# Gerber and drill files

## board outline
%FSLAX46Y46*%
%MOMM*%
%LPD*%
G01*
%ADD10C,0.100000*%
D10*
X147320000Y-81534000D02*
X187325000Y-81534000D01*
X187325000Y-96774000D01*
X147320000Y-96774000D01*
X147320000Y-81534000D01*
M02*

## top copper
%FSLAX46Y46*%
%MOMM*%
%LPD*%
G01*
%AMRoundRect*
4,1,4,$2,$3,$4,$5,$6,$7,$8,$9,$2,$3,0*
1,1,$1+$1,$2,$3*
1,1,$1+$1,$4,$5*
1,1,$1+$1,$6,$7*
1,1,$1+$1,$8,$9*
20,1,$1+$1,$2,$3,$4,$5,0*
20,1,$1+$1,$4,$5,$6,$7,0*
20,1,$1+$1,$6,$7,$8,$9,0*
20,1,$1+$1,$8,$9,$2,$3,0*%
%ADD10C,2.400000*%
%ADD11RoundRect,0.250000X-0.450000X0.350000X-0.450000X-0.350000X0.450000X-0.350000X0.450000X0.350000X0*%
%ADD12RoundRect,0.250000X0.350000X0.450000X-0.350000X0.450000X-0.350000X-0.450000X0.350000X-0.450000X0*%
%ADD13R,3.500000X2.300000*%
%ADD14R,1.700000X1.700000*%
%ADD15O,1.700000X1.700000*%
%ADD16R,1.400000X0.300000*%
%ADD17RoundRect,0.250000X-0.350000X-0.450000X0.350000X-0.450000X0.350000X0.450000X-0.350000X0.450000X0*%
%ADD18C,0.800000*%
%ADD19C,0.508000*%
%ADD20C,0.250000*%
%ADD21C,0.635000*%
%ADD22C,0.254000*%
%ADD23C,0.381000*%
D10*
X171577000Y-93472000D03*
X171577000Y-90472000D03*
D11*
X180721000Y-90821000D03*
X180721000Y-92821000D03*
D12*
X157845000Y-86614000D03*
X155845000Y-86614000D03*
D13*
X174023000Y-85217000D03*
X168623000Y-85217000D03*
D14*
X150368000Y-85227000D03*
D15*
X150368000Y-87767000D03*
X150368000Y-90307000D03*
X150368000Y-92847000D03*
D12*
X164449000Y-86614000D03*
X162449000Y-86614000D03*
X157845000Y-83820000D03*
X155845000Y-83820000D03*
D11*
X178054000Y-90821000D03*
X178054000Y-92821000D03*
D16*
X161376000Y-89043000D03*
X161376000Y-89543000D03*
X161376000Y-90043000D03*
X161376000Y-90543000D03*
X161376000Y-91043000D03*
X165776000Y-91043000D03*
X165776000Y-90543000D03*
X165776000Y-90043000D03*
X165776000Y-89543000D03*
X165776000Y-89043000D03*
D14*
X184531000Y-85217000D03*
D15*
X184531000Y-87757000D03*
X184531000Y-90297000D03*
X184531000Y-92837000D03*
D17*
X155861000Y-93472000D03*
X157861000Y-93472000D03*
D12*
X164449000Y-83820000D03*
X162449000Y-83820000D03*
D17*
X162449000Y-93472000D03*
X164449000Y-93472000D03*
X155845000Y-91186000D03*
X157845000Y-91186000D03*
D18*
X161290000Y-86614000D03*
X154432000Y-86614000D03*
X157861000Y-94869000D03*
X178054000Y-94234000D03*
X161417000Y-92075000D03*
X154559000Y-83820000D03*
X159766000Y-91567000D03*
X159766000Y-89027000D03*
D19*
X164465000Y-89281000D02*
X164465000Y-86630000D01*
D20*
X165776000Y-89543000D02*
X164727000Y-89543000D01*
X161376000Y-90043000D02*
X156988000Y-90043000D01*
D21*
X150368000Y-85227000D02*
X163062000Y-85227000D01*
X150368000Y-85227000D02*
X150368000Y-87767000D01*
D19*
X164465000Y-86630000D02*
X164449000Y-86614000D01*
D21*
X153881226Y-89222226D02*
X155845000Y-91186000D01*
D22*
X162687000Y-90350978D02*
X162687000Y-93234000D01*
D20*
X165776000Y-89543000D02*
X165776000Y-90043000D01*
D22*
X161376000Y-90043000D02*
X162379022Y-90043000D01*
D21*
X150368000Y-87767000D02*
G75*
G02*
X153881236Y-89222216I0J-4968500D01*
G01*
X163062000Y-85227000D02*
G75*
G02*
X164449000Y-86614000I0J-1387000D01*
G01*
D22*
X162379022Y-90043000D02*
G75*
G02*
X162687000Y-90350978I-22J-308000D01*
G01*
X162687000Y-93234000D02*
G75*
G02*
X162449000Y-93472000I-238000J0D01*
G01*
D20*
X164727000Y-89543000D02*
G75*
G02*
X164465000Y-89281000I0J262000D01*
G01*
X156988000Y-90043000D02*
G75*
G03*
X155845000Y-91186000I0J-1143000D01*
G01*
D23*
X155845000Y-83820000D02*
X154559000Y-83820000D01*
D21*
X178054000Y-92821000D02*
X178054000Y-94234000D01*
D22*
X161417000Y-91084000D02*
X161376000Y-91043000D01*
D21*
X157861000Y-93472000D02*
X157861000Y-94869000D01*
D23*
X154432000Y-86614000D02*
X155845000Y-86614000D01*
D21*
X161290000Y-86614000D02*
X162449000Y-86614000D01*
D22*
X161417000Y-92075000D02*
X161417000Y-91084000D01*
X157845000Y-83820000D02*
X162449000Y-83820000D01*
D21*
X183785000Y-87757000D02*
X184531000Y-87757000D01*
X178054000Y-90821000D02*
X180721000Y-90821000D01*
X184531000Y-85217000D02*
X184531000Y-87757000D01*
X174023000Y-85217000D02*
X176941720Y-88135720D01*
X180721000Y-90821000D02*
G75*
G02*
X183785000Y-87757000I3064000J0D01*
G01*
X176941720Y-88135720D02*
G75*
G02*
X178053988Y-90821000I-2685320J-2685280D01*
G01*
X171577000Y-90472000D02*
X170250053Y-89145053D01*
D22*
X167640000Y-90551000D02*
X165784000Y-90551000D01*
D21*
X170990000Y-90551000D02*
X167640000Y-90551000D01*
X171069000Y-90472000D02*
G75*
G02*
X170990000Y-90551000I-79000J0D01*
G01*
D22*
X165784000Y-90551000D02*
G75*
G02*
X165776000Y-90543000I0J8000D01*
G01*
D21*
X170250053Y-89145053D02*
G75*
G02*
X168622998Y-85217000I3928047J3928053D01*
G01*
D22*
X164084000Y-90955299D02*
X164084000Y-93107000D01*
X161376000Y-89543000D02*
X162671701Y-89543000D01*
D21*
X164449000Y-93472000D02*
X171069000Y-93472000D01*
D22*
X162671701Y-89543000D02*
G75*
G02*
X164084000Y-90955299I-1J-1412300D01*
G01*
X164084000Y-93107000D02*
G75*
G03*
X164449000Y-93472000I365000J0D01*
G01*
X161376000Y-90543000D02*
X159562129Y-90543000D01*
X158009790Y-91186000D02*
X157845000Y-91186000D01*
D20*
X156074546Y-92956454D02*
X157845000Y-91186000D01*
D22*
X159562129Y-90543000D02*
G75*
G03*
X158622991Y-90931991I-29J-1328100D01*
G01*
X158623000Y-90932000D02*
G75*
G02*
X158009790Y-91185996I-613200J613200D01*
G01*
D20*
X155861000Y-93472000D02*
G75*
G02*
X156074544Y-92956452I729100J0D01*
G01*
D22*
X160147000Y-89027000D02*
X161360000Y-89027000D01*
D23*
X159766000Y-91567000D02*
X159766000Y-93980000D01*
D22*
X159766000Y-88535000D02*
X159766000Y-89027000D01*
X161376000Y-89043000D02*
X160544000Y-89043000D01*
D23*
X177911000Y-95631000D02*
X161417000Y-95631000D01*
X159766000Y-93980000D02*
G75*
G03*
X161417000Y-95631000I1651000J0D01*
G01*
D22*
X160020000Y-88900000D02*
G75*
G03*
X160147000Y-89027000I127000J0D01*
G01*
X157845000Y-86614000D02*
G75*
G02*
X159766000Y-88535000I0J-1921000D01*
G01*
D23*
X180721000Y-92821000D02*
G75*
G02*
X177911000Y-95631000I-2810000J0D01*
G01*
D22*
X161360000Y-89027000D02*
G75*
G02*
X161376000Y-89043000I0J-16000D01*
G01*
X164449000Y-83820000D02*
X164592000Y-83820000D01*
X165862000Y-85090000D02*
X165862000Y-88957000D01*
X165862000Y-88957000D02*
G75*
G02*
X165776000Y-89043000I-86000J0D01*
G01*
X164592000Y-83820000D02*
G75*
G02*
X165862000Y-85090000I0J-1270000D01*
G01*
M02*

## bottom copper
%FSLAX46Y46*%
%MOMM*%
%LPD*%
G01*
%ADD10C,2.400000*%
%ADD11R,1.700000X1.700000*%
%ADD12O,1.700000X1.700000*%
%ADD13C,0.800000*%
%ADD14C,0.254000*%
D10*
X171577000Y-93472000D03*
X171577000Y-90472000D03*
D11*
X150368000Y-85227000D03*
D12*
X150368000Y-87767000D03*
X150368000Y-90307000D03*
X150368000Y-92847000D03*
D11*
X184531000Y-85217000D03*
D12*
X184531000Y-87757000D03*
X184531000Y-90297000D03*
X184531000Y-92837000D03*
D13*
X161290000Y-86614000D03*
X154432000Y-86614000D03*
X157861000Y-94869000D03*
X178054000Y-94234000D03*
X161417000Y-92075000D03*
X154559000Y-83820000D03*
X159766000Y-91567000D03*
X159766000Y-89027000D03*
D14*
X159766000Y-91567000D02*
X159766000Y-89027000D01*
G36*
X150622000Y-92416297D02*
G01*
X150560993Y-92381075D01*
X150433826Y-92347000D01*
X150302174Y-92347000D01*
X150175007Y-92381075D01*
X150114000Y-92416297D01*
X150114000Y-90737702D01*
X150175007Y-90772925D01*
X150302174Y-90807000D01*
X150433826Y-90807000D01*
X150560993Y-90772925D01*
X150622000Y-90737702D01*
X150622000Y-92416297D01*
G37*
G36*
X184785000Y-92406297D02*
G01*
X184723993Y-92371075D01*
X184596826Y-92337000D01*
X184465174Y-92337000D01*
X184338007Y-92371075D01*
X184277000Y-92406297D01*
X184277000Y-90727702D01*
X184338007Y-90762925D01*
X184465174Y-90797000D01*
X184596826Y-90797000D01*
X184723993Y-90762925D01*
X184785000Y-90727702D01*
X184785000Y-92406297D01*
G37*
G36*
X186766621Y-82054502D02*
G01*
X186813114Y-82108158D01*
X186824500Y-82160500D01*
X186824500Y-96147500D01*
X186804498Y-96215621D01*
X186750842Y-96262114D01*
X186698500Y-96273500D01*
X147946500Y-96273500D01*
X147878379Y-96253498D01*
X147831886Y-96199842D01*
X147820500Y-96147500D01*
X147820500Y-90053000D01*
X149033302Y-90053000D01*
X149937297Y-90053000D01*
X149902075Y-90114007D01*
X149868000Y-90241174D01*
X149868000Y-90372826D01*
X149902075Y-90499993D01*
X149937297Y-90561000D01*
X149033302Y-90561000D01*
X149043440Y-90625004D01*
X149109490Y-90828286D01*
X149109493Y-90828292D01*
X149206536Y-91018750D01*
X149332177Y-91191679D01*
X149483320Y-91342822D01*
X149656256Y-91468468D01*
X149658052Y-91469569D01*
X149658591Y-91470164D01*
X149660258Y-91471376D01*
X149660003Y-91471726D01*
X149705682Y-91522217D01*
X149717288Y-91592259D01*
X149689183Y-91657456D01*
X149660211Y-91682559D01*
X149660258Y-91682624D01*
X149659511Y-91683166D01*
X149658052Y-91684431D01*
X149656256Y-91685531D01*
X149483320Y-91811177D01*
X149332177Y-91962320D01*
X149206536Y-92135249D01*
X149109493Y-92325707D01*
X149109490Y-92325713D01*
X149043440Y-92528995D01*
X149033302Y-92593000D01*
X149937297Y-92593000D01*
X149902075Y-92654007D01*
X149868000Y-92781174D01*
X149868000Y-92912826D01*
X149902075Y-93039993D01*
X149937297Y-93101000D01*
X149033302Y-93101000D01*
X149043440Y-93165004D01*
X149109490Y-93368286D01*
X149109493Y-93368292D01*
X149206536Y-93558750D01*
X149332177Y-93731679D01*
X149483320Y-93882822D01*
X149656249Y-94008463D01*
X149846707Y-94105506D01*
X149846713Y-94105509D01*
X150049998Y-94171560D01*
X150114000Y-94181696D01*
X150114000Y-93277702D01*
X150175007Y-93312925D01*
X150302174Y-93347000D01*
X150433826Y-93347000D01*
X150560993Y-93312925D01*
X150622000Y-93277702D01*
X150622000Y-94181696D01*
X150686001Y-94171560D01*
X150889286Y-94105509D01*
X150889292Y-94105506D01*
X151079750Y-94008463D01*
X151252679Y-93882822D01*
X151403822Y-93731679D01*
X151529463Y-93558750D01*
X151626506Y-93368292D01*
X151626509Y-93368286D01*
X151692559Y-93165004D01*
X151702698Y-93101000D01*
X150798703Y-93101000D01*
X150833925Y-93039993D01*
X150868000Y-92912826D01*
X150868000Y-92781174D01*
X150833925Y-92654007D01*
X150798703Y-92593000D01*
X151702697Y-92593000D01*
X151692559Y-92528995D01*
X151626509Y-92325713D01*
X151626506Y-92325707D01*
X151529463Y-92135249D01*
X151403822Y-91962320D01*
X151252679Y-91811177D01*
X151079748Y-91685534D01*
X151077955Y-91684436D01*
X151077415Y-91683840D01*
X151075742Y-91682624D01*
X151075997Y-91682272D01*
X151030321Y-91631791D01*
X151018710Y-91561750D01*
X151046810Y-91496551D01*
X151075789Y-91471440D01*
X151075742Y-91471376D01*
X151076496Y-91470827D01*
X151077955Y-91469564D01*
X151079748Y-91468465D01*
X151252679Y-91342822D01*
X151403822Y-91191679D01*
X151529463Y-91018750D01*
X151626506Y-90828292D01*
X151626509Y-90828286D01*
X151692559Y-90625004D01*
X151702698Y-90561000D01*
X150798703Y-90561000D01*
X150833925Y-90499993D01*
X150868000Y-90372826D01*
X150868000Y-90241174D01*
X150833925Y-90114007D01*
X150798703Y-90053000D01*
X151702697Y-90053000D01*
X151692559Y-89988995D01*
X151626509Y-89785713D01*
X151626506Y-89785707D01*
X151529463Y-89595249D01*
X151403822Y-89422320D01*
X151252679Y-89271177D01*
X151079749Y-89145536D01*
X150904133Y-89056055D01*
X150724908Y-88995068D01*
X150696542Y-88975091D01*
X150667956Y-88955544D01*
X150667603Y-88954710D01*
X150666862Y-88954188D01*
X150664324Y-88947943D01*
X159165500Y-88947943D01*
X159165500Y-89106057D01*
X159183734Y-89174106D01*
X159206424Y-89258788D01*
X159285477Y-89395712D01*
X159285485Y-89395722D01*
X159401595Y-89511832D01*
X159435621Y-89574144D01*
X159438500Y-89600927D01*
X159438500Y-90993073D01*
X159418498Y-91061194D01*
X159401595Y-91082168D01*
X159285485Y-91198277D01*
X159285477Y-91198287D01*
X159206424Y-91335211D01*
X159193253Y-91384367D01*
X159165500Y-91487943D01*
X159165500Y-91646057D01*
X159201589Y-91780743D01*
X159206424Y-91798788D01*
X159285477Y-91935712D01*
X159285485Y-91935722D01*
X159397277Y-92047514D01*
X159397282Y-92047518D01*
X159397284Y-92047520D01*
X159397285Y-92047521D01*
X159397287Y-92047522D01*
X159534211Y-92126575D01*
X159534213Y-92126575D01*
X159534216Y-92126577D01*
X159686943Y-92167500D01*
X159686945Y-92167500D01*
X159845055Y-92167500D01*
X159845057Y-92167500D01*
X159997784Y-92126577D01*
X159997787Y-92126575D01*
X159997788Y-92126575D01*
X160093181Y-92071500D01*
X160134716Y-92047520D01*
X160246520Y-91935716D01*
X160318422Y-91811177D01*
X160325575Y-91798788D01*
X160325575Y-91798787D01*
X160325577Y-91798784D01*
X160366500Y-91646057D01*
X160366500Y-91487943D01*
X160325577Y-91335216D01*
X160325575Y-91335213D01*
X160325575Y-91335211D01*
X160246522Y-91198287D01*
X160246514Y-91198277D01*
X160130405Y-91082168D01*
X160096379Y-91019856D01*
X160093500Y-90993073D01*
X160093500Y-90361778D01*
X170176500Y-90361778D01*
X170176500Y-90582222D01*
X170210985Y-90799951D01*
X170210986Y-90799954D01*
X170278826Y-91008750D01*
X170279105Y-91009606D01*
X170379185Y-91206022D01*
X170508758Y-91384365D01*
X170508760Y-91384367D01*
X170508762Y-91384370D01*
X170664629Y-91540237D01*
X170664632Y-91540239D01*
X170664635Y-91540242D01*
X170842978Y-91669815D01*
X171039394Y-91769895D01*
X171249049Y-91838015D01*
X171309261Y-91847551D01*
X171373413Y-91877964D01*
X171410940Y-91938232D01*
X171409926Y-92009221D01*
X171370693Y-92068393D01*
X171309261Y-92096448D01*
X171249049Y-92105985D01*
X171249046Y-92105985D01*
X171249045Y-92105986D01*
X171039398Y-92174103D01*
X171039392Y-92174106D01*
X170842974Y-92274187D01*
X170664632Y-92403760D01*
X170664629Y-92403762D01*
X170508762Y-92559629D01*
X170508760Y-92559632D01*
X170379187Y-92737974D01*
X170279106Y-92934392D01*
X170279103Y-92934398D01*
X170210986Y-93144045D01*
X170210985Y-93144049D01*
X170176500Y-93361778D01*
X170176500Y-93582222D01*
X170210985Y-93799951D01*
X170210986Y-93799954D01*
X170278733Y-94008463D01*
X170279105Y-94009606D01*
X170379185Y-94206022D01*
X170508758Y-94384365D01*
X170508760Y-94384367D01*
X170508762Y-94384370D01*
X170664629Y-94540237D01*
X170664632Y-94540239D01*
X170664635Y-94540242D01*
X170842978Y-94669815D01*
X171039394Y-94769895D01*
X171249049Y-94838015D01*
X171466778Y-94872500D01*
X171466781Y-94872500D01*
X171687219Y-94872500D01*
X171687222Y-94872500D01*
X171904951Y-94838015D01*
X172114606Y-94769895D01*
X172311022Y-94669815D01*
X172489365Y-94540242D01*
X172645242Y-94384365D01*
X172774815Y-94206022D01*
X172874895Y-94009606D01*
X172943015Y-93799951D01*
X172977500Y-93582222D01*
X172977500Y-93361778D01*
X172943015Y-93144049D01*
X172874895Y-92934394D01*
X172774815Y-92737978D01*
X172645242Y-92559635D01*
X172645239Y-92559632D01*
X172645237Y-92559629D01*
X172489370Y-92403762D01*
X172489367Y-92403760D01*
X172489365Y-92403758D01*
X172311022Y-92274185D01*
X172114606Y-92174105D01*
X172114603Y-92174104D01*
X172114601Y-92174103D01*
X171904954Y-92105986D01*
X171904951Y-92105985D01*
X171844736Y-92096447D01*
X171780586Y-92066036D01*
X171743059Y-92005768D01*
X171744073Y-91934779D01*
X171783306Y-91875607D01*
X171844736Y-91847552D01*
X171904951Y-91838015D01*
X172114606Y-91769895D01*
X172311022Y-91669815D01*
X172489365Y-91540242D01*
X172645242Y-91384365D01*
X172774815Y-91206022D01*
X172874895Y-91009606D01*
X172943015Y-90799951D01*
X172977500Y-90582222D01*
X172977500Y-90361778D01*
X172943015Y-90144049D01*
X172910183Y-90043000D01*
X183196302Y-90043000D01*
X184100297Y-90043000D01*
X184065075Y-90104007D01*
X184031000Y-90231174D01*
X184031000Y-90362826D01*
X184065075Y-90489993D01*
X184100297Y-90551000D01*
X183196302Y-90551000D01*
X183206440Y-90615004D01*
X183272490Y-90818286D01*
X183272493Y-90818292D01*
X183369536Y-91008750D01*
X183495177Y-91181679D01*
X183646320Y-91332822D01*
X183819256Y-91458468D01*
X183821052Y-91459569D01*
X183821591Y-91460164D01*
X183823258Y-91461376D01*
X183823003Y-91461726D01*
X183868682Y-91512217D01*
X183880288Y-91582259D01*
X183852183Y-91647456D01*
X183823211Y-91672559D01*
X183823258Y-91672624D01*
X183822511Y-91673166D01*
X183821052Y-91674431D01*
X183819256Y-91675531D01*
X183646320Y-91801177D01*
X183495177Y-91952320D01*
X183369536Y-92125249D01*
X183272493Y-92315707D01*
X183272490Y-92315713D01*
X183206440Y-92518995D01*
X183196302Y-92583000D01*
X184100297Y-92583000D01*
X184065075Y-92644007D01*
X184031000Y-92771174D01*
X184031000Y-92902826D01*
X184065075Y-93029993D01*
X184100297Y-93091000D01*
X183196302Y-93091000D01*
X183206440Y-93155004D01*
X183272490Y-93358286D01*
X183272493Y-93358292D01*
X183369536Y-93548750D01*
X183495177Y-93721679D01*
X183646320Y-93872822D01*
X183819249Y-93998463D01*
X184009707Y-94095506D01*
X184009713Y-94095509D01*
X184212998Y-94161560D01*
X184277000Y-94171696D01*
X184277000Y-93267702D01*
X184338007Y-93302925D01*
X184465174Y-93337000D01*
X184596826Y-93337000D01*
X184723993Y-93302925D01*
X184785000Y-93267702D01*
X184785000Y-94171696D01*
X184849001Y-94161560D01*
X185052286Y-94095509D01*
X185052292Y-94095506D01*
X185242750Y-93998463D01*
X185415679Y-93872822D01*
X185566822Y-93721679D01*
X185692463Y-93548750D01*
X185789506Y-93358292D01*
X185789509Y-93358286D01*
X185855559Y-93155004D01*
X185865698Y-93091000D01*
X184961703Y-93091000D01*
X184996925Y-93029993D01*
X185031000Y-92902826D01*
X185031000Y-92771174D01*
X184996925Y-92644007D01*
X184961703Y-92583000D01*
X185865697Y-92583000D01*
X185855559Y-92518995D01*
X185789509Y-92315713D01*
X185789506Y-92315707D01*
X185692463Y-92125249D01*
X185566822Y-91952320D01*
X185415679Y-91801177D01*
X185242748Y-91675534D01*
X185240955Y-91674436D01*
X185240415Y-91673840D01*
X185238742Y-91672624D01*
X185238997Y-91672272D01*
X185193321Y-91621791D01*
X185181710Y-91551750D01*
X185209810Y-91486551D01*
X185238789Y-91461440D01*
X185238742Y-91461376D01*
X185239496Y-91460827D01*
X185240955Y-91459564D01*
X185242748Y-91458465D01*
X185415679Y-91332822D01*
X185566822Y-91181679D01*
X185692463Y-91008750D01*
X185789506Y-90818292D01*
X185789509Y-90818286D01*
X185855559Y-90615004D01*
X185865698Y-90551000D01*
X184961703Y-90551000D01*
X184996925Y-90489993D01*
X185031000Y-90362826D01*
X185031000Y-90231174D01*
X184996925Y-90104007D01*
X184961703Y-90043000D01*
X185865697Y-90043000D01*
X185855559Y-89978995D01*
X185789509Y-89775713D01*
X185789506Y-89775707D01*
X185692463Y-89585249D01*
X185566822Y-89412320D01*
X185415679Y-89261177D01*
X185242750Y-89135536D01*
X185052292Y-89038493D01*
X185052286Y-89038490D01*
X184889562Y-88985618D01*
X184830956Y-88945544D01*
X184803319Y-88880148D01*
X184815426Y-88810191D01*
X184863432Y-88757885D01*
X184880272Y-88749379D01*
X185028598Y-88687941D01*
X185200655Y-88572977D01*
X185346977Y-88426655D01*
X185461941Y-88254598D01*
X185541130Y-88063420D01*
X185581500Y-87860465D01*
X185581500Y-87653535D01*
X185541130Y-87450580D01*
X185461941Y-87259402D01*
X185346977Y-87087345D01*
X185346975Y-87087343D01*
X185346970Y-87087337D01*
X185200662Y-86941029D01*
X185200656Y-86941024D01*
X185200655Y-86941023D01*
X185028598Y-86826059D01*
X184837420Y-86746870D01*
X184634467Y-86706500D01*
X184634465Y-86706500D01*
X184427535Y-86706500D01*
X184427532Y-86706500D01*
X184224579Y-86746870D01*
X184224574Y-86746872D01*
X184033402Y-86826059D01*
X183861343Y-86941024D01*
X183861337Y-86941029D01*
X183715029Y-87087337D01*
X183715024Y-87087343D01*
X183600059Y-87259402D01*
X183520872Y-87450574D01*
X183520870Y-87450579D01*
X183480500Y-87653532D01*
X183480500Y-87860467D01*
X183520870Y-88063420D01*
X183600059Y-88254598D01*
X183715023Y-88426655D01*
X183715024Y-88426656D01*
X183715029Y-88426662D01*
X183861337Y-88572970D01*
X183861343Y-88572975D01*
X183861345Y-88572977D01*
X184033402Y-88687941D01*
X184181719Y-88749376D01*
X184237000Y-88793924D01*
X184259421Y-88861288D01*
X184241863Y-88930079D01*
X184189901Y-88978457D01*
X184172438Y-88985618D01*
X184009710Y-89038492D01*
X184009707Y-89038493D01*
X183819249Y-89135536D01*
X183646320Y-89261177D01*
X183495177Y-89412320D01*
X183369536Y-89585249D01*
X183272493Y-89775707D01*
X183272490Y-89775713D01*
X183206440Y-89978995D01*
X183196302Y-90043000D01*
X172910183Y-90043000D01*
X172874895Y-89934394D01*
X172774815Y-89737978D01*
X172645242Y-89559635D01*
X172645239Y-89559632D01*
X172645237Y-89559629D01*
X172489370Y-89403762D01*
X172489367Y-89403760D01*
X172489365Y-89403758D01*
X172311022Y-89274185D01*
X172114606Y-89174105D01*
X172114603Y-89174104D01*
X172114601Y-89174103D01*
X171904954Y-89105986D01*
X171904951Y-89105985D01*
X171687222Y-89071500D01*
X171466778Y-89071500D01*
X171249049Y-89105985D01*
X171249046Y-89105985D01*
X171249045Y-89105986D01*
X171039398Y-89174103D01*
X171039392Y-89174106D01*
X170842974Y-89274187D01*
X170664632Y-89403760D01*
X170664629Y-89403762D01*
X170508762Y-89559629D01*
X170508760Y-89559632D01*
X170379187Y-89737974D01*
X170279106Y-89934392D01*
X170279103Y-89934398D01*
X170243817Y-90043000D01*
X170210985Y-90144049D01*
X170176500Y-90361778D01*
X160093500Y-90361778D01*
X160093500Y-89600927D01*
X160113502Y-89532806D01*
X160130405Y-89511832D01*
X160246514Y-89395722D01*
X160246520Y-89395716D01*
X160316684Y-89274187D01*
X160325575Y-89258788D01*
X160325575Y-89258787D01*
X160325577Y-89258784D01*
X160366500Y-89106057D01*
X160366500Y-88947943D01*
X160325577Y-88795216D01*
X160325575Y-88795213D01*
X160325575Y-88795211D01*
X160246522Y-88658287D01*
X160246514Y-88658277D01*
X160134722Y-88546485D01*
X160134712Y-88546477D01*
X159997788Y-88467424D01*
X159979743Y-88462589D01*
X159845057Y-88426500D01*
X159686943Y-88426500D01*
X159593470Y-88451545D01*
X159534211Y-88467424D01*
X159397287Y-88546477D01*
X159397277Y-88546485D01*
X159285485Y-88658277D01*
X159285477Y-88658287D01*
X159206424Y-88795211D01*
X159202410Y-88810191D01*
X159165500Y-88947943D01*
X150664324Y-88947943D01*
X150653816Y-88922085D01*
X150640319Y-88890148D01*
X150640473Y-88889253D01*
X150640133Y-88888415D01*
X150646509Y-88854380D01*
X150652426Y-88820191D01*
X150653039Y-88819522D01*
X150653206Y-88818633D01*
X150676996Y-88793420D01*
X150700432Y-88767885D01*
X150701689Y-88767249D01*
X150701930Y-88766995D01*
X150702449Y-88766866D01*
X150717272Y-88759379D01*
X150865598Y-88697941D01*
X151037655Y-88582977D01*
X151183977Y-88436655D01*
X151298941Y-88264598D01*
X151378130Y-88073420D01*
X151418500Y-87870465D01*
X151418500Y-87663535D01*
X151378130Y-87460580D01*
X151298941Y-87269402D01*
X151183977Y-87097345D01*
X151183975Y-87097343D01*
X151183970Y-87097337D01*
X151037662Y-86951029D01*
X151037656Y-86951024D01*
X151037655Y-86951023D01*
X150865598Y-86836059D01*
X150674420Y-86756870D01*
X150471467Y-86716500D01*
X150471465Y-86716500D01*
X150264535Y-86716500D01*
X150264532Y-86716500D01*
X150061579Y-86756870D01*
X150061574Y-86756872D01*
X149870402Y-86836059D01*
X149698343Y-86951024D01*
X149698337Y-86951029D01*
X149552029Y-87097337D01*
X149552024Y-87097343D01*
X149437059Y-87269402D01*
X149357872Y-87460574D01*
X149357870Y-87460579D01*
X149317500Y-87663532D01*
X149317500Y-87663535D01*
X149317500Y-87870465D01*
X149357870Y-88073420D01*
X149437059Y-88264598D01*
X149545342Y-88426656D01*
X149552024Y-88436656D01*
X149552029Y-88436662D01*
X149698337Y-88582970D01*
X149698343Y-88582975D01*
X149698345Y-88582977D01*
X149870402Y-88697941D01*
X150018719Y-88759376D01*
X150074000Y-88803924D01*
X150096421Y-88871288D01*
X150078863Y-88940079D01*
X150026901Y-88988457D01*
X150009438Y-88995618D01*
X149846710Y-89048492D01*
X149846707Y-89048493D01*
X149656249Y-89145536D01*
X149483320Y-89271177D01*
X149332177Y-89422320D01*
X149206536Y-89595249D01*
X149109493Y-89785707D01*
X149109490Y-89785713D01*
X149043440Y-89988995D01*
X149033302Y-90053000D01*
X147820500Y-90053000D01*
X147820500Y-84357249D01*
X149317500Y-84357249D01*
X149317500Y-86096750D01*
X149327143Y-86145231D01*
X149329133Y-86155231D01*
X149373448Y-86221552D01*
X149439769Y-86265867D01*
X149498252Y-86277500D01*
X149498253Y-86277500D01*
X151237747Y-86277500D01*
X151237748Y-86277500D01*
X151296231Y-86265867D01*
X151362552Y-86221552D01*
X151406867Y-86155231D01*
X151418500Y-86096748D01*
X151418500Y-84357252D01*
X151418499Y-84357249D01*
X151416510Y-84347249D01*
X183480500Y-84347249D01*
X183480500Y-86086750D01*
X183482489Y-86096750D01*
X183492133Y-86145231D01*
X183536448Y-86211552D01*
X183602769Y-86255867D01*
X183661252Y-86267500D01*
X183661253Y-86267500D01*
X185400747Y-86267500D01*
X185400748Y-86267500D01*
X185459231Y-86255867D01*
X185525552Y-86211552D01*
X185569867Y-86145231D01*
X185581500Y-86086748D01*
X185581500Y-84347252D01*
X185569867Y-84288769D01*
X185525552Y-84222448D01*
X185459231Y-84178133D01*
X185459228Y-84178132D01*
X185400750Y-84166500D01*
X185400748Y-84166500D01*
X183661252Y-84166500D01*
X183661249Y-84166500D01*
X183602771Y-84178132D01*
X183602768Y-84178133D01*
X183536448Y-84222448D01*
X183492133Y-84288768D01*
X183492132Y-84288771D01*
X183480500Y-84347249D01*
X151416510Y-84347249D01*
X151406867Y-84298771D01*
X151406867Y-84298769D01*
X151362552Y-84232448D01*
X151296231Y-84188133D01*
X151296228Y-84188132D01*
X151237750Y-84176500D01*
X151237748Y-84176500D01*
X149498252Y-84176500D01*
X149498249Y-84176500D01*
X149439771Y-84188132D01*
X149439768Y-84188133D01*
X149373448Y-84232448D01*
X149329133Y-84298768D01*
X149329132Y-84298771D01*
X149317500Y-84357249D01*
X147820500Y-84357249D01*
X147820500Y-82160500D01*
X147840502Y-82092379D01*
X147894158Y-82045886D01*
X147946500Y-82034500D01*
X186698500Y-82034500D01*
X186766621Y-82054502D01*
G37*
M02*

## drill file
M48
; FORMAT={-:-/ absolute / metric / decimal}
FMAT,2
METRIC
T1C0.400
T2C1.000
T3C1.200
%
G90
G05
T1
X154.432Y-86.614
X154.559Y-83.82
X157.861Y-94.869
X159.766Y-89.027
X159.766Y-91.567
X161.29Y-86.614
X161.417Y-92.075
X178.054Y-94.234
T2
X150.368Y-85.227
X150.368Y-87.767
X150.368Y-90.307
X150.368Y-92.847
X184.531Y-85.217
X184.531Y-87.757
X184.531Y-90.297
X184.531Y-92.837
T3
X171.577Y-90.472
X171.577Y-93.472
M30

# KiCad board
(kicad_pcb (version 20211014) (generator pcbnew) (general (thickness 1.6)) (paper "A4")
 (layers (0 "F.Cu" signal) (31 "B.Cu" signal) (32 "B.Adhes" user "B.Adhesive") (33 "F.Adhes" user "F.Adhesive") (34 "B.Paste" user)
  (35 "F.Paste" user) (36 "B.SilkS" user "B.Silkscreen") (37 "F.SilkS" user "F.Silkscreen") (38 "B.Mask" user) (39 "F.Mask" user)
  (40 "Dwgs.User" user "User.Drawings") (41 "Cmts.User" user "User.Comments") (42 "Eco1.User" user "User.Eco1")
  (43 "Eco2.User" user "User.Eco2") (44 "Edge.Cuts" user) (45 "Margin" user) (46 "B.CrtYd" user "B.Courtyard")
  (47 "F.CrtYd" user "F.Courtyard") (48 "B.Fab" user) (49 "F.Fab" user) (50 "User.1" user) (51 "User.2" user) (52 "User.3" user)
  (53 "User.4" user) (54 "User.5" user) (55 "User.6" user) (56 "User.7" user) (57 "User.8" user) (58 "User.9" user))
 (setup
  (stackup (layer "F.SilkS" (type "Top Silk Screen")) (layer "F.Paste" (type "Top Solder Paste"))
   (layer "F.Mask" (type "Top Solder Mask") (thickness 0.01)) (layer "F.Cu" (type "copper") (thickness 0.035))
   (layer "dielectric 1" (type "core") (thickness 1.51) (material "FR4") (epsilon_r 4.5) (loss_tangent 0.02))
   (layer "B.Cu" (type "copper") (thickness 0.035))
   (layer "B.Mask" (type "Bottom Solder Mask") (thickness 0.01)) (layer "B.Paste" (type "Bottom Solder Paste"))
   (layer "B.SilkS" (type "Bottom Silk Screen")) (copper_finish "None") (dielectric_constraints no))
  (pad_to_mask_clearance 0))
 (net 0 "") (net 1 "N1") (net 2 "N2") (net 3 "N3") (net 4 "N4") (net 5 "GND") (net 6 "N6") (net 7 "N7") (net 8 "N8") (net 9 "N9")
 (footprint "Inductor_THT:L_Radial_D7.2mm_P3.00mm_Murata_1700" (layer "F.Cu") (at 171.577 93.472 90)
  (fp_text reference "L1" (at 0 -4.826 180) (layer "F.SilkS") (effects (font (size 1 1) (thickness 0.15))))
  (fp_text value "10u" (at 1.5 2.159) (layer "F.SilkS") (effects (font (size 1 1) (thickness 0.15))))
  (pad "1" thru_hole circle (at 0 0 90) (size 2.4 2.4) (drill 1.2) (layers *.Cu *.Mask) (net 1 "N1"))
  (pad "2" thru_hole circle (at 3 0 90) (size 2.4 2.4) (drill 1.2) (layers *.Cu *.Mask) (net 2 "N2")))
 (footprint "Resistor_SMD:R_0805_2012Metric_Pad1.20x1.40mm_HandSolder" (layer "F.Cu") (at 180.721 91.821 -90)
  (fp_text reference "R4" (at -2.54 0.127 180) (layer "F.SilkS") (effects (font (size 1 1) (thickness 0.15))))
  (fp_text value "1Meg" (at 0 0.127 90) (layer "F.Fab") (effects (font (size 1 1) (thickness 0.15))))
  (pad "1" smd roundrect (at -1 0 270) (size 1.2 1.4) (layers "F.Cu" "F.Paste" "F.Mask") (roundrect_rratio 0.208333) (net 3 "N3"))
  (pad "2" smd roundrect (at 1 0 270) (size 1.2 1.4) (layers "F.Cu" "F.Paste" "F.Mask") (roundrect_rratio 0.208333) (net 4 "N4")))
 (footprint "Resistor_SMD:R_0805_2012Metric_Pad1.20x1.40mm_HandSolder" (layer "F.Cu") (at 156.845 86.614 180)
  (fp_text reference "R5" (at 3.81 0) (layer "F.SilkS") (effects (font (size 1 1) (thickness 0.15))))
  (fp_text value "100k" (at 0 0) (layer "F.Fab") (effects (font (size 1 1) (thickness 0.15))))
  (pad "1" smd roundrect (at -1 0 180) (size 1.2 1.4) (layers "F.Cu" "F.Paste" "F.Mask") (roundrect_rratio 0.208333) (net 4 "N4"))
  (pad "2" smd roundrect (at 1 0 180) (size 1.2 1.4) (layers "F.Cu" "F.Paste" "F.Mask") (roundrect_rratio 0.208333) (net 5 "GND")))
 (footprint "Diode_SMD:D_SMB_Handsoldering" (layer "F.Cu") (at 171.323 85.217 180)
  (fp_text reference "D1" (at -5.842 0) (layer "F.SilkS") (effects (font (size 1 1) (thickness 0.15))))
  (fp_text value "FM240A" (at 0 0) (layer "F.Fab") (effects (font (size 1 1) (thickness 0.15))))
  (pad "1" smd rect (at -2.7 0 180) (size 3.5 2.3) (layers "F.Cu" "F.Paste" "F.Mask") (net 3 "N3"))
  (pad "2" smd rect (at 2.7 0 180) (size 3.5 2.3) (layers "F.Cu" "F.Paste" "F.Mask") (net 2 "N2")))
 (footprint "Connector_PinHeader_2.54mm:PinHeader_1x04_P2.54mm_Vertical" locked (layer "F.Cu") (at 150.368 85.227)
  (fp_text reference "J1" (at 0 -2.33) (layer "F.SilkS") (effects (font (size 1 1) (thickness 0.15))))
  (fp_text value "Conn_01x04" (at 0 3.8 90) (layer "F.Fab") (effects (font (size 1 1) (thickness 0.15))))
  (pad "1" thru_hole rect locked (at 0 0) (size 1.7 1.7) (drill 1) (layers *.Cu *.Mask) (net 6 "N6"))
  (pad "2" thru_hole oval locked (at 0 2.54) (size 1.7 1.7) (drill 1) (layers *.Cu *.Mask) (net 6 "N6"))
  (pad "3" thru_hole oval locked (at 0 5.08) (size 1.7 1.7) (drill 1) (layers *.Cu *.Mask) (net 5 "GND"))
  (pad "4" thru_hole oval locked (at 0 7.62) (size 1.7 1.7) (drill 1) (layers *.Cu *.Mask) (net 5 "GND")))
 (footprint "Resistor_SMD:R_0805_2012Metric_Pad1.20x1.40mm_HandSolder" (layer "F.Cu") (at 163.449 86.614 180)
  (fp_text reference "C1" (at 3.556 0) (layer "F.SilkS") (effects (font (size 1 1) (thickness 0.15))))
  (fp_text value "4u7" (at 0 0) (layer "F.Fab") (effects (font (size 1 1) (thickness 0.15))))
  (pad "1" smd roundrect (at -1 0 180) (size 1.2 1.4) (layers "F.Cu" "F.Paste" "F.Mask") (roundrect_rratio 0.208333) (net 6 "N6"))
  (pad "2" smd roundrect (at 1 0 180) (size 1.2 1.4) (layers "F.Cu" "F.Paste" "F.Mask") (roundrect_rratio 0.208333) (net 5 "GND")))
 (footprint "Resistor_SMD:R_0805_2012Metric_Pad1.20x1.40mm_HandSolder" (layer "F.Cu") (at 156.845 83.82 180)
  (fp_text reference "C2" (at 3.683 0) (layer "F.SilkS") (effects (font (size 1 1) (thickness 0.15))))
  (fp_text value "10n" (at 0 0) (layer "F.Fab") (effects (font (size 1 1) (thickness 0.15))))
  (pad "1" smd roundrect (at -1 0 180) (size 1.2 1.4) (layers "F.Cu" "F.Paste" "F.Mask") (roundrect_rratio 0.208333) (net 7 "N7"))
  (pad "2" smd roundrect (at 1 0 180) (size 1.2 1.4) (layers "F.Cu" "F.Paste" "F.Mask") (roundrect_rratio 0.208333) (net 5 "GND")))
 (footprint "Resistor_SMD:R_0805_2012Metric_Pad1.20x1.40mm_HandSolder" (layer "F.Cu") (at 178.054 91.821 -90)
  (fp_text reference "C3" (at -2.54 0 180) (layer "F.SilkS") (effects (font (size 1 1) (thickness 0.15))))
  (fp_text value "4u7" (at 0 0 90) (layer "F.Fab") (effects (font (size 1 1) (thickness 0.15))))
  (pad "1" smd roundrect (at -1 0 270) (size 1.2 1.4) (layers "F.Cu" "F.Paste" "F.Mask") (roundrect_rratio 0.208333) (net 3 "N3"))
  (pad "2" smd roundrect (at 1 0 270) (size 1.2 1.4) (layers "F.Cu" "F.Paste" "F.Mask") (roundrect_rratio 0.208333) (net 5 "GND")))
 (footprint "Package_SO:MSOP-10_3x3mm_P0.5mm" (layer "F.Cu") (at 163.576 90.043)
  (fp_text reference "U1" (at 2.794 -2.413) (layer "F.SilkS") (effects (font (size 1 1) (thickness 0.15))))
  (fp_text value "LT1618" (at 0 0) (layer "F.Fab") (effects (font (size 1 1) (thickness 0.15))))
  (pad "1" smd rect (at -2.2 -1) (size 1.4 0.3) (layers "F.Cu" "F.Paste" "F.Mask") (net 4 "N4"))
  (pad "2" smd rect (at -2.2 -0.5) (size 1.4 0.3) (layers "F.Cu" "F.Paste" "F.Mask") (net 1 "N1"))
  (pad "3" smd rect (at -2.2 0) (size 1.4 0.3) (layers "F.Cu" "F.Paste" "F.Mask") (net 6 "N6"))
  (pad "4" smd rect (at -2.2 0.5) (size 1.4 0.3) (layers "F.Cu" "F.Paste" "F.Mask") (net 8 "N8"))
  (pad "5" smd rect (at -2.2 1) (size 1.4 0.3) (layers "F.Cu" "F.Paste" "F.Mask") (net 5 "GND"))
  (pad "6" smd rect (at 2.2 1) (size 1.4 0.3) (layers "F.Cu" "F.Paste" "F.Mask"))
  (pad "7" smd rect (at 2.2 0.5) (size 1.4 0.3) (layers "F.Cu" "F.Paste" "F.Mask") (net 2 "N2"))
  (pad "8" smd rect (at 2.2 0) (size 1.4 0.3) (layers "F.Cu" "F.Paste" "F.Mask") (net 6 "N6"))
  (pad "9" smd rect (at 2.2 -0.5) (size 1.4 0.3) (layers "F.Cu" "F.Paste" "F.Mask") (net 6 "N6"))
  (pad "10" smd rect (at 2.2 -1) (size 1.4 0.3) (layers "F.Cu" "F.Paste" "F.Mask") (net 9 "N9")))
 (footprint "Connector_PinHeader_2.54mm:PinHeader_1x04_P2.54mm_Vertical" (layer "F.Cu") (at 184.531 85.217)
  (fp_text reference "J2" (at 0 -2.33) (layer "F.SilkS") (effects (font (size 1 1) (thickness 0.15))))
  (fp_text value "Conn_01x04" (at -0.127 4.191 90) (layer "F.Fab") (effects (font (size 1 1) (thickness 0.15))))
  (pad "1" thru_hole rect (at 0 0) (size 1.7 1.7) (drill 1) (layers *.Cu *.Mask) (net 3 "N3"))
  (pad "2" thru_hole oval (at 0 2.54) (size 1.7 1.7) (drill 1) (layers *.Cu *.Mask) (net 3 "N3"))
  (pad "3" thru_hole oval (at 0 5.08) (size 1.7 1.7) (drill 1) (layers *.Cu *.Mask) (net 5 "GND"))
  (pad "4" thru_hole oval (at 0 7.62) (size 1.7 1.7) (drill 1) (layers *.Cu *.Mask) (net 5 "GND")))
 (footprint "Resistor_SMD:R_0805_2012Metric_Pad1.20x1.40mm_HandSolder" (layer "F.Cu") (at 156.861 93.472)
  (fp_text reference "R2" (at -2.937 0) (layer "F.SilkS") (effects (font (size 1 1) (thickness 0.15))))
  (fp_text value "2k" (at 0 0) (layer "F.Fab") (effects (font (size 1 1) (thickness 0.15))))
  (pad "1" smd roundrect (at -1 0) (size 1.2 1.4) (layers "F.Cu" "F.Paste" "F.Mask") (roundrect_rratio 0.208333) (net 8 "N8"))
  (pad "2" smd roundrect (at 1 0) (size 1.2 1.4) (layers "F.Cu" "F.Paste" "F.Mask") (roundrect_rratio 0.208333) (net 5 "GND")))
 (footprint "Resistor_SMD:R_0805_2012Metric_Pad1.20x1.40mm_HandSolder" (layer "F.Cu") (at 163.449 83.82 180)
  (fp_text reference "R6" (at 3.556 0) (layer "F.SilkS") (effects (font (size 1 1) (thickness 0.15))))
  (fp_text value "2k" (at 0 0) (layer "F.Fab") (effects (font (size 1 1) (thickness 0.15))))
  (pad "1" smd roundrect (at -1 0 180) (size 1.2 1.4) (layers "F.Cu" "F.Paste" "F.Mask") (roundrect_rratio 0.208333) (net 9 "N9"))
  (pad "2" smd roundrect (at 1 0 180) (size 1.2 1.4) (layers "F.Cu" "F.Paste" "F.Mask") (roundrect_rratio 0.208333) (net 7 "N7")))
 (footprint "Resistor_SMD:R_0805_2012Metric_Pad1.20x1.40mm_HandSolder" (layer "F.Cu") (at 163.449 93.472)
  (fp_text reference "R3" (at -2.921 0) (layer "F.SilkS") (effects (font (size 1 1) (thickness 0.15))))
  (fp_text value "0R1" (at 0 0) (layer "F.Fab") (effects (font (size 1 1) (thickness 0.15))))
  (pad "1" smd roundrect (at -1 0) (size 1.2 1.4) (layers "F.Cu" "F.Paste" "F.Mask") (roundrect_rratio 0.208333) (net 6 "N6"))
  (pad "2" smd roundrect (at 1 0) (size 1.2 1.4) (layers "F.Cu" "F.Paste" "F.Mask") (roundrect_rratio 0.208333) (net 1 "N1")))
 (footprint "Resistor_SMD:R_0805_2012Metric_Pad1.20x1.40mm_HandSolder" (layer "F.Cu") (at 156.845 91.186)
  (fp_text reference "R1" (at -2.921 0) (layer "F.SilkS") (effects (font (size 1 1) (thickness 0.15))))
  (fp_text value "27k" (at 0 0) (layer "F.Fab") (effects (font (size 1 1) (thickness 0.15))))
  (pad "1" smd roundrect (at -1 0) (size 1.2 1.4) (layers "F.Cu" "F.Paste" "F.Mask") (roundrect_rratio 0.208333) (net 6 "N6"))
  (pad "2" smd roundrect (at 1 0) (size 1.2 1.4) (layers "F.Cu" "F.Paste" "F.Mask") (roundrect_rratio 0.208333) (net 8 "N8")))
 (gr_rect (start 147.32 96.774) (end 187.325 81.534) (layer "Edge.Cuts") (width 0.1) (fill none))
 (segment (start 164.465 89.281) (end 164.465 86.63) (width 0.508) (layer "F.Cu") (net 6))
 (segment (start 165.776 89.543) (end 164.727 89.543) (width 0.25) (layer "F.Cu") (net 6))
 (segment (start 161.376 90.043) (end 156.988 90.043) (width 0.25) (layer "F.Cu") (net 6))
 (segment (start 150.368 85.227) (end 163.062 85.227) (width 0.635) (layer "F.Cu") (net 6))
 (segment (start 150.368 85.227) (end 150.368 87.767) (width 0.635) (layer "F.Cu") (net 6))
 (segment (start 164.465 86.63) (end 164.449 86.614) (width 0.508) (layer "F.Cu") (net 6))
 (segment (start 153.881226 89.222226) (end 155.845 91.186) (width 0.635) (layer "F.Cu") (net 6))
 (segment (start 162.687 90.350978) (end 162.687 93.234) (width 0.254) (layer "F.Cu") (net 6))
 (segment (start 165.776 89.543) (end 165.776 90.043) (width 0.25) (layer "F.Cu") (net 6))
 (segment (start 161.376 90.043) (end 162.379022 90.043) (width 0.254) (layer "F.Cu") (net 6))
 (arc (start 150.368 87.767) (mid 152.269344 88.145201) (end 153.881226 89.222226) (width 0.635) (layer "F.Cu") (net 6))
 (arc (start 163.062 85.227) (mid 164.042757 85.633243) (end 164.449 86.614) (width 0.635) (layer "F.Cu") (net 6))
 (arc (start 162.379022 90.043) (mid 162.596795 90.133205) (end 162.687 90.350978) (width 0.254) (layer "F.Cu") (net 6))
 (arc (start 162.687 93.234) (mid 162.617291 93.402291) (end 162.449 93.472) (width 0.254) (layer "F.Cu") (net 6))
 (arc (start 164.727 89.543) (mid 164.541738 89.466262) (end 164.465 89.281) (width 0.25) (layer "F.Cu") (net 6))
 (arc (start 156.988 90.043) (mid 156.179777 90.377777) (end 155.845 91.186) (width 0.25) (layer "F.Cu") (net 6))
 (segment (start 155.845 83.82) (end 154.559 83.82) (width 0.381) (layer "F.Cu") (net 5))
 (segment (start 178.054 92.821) (end 178.054 94.234) (width 0.635) (layer "F.Cu") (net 5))
 (segment (start 161.417 91.084) (end 161.376 91.043) (width 0.254) (layer "F.Cu") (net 5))
 (segment (start 157.861 93.472) (end 157.861 94.869) (width 0.635) (layer "F.Cu") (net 5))
 (segment (start 154.432 86.614) (end 155.845 86.614) (width 0.381) (layer "F.Cu") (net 5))
 (segment (start 161.29 86.614) (end 162.449 86.614) (width 0.635) (layer "F.Cu") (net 5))
 (segment (start 161.417 92.075) (end 161.417 91.084) (width 0.254) (layer "F.Cu") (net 5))
 (via (at 161.29 86.614) (size 0.8) (drill 0.4) (layers "F.Cu" "B.Cu") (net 5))
 (via (at 154.432 86.614) (size 0.8) (drill 0.4) (layers "F.Cu" "B.Cu") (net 5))
 (via (at 157.861 94.869) (size 0.8) (drill 0.4) (layers "F.Cu" "B.Cu") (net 5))
 (via (at 178.054 94.234) (size 0.8) (drill 0.4) (layers "F.Cu" "B.Cu") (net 5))
 (via (at 161.417 92.075) (size 0.8) (drill 0.4) (layers "F.Cu" "B.Cu") (free) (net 5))
 (via (at 154.559 83.82) (size 0.8) (drill 0.4) (layers "F.Cu" "B.Cu") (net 5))
 (segment (start 157.845 83.82) (end 162.449 83.82) (width 0.254) (layer "F.Cu") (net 7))
 (segment (start 183.785 87.757) (end 184.531 87.757) (width 0.635) (layer "F.Cu") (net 3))
 (segment (start 178.054 90.821) (end 180.721 90.821) (width 0.635) (layer "F.Cu") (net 3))
 (segment (start 184.531 85.217) (end 184.531 87.757) (width 0.635) (layer "F.Cu") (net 3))
 (segment (start 174.023 85.217) (end 176.94172 88.13572) (width 0.635) (layer "F.Cu") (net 3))
 (arc (start 180.721 90.821) (mid 181.618425 88.654425) (end 183.785 87.757) (width 0.635) (layer "F.Cu") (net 3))
 (arc (start 176.94172 88.13572) (mid 177.764927 89.367737) (end 178.054 90.821) (width 0.635) (layer "F.Cu") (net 3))
 (segment (start 171.577 90.472) (end 170.250053 89.145053) (width 0.635) (layer "F.Cu") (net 2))
 (segment (start 167.64 90.551) (end 165.784 90.551) (width 0.254) (layer "F.Cu") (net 2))
 (segment (start 170.99 90.551) (end 167.64 90.551) (width 0.635) (layer "F.Cu") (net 2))
 (arc (start 171.069 90.472) (mid 171.045861 90.527861) (end 170.99 90.551) (width 0.635) (layer "F.Cu") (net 2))
 (arc (start 165.784 90.551) (mid 165.778343 90.548657) (end 165.776 90.543) (width 0.254) (layer "F.Cu") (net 2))
 (arc (start 170.250053 89.145053) (mid 169.045857 87.342847) (end 168.623 85.217) (width 0.635) (layer "F.Cu") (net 2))
 (segment (start 164.084 90.955299) (end 164.084 93.107) (width 0.254) (layer "F.Cu") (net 1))
 (segment (start 161.376 89.543) (end 162.671701 89.543) (width 0.254) (layer "F.Cu") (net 1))
 (segment (start 164.449 93.472) (end 171.069 93.472) (width 0.635) (layer "F.Cu") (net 1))
 (arc (start 162.671701 89.543) (mid 163.670347 89.956653) (end 164.084 90.955299) (width 0.254) (layer "F.Cu") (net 1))
 (arc (start 164.084 93.107) (mid 164.190906 93.365094) (end 164.449 93.472) (width 0.254) (layer "F.Cu") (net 1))
 (segment (start 161.376 90.543) (end 159.562129 90.543) (width 0.254) (layer "F.Cu") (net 8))
 (segment (start 158.00979 91.186) (end 157.845 91.186) (width 0.254) (layer "F.Cu") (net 8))
 (segment (start 156.074546 92.956454) (end 157.845 91.186) (width 0.25) (layer "F.Cu") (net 8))
 (arc (start 159.562129 90.543) (mid 159.053876 90.644098) (end 158.623 90.932) (width 0.254) (layer "F.Cu") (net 8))
 (arc (start 158.623 90.932) (mid 158.341657 91.119988) (end 158.00979 91.186) (width 0.254) (layer "F.Cu") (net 8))
 (arc (start 155.861 93.472) (mid 155.916499 93.192989) (end 156.074546 92.956454) (width 0.25) (layer "F.Cu") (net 8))
 (segment (start 160.147 89.027) (end 161.36 89.027) (width 0.254) (layer "F.Cu") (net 4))
 (segment (start 159.766 91.567) (end 159.766 93.98) (width 0.381) (layer "F.Cu") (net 4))
 (segment (start 159.766 88.535) (end 159.766 89.027) (width 0.254) (layer "F.Cu") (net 4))
 (segment (start 161.376 89.043) (end 160.544 89.043) (width 0.254) (layer "F.Cu") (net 4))
 (segment (start 177.911 95.631) (end 161.417 95.631) (width 0.381) (layer "F.Cu") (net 4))
 (via (at 159.766 91.567) (size 0.8) (drill 0.4) (layers "F.Cu" "B.Cu") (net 4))
 (via (at 159.766 89.027) (size 0.8) (drill 0.4) (layers "F.Cu" "B.Cu") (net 4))
 (arc (start 159.766 93.98) (mid 160.249567 95.147433) (end 161.417 95.631) (width 0.381) (layer "F.Cu") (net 4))
 (arc (start 160.02 88.9) (mid 160.057197 88.989803) (end 160.147 89.027) (width 0.254) (layer "F.Cu") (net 4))
 (arc (start 157.845 86.614) (mid 159.203352 87.176648) (end 159.766 88.535) (width 0.254) (layer "F.Cu") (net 4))
 (arc (start 180.721 92.821) (mid 179.89797 94.80797) (end 177.911 95.631) (width 0.381) (layer "F.Cu") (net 4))
 (arc (start 161.36 89.027) (mid 161.371314 89.031686) (end 161.376 89.043) (width 0.254) (layer "F.Cu") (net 4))
 (segment (start 159.766 91.567) (end 159.766 89.027) (width 0.254) (layer "B.Cu") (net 4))
 (segment (start 164.449 83.82) (end 164.592 83.82) (width 0.254) (layer "F.Cu") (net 9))
 (segment (start 165.862 85.09) (end 165.862 88.957) (width 0.254) (layer "F.Cu") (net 9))
 (arc (start 165.862 88.957) (mid 165.836811 89.017811) (end 165.776 89.043) (width 0.254) (layer "F.Cu") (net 9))
 (arc (start 164.592 83.82) (mid 165.490026 84.191974) (end 165.862 85.09) (width 0.254) (layer "F.Cu") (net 9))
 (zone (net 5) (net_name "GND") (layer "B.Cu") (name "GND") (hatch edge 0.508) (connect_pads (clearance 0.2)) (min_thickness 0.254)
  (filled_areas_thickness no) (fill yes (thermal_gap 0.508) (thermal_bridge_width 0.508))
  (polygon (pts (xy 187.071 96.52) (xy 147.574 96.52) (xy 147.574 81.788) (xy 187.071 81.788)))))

